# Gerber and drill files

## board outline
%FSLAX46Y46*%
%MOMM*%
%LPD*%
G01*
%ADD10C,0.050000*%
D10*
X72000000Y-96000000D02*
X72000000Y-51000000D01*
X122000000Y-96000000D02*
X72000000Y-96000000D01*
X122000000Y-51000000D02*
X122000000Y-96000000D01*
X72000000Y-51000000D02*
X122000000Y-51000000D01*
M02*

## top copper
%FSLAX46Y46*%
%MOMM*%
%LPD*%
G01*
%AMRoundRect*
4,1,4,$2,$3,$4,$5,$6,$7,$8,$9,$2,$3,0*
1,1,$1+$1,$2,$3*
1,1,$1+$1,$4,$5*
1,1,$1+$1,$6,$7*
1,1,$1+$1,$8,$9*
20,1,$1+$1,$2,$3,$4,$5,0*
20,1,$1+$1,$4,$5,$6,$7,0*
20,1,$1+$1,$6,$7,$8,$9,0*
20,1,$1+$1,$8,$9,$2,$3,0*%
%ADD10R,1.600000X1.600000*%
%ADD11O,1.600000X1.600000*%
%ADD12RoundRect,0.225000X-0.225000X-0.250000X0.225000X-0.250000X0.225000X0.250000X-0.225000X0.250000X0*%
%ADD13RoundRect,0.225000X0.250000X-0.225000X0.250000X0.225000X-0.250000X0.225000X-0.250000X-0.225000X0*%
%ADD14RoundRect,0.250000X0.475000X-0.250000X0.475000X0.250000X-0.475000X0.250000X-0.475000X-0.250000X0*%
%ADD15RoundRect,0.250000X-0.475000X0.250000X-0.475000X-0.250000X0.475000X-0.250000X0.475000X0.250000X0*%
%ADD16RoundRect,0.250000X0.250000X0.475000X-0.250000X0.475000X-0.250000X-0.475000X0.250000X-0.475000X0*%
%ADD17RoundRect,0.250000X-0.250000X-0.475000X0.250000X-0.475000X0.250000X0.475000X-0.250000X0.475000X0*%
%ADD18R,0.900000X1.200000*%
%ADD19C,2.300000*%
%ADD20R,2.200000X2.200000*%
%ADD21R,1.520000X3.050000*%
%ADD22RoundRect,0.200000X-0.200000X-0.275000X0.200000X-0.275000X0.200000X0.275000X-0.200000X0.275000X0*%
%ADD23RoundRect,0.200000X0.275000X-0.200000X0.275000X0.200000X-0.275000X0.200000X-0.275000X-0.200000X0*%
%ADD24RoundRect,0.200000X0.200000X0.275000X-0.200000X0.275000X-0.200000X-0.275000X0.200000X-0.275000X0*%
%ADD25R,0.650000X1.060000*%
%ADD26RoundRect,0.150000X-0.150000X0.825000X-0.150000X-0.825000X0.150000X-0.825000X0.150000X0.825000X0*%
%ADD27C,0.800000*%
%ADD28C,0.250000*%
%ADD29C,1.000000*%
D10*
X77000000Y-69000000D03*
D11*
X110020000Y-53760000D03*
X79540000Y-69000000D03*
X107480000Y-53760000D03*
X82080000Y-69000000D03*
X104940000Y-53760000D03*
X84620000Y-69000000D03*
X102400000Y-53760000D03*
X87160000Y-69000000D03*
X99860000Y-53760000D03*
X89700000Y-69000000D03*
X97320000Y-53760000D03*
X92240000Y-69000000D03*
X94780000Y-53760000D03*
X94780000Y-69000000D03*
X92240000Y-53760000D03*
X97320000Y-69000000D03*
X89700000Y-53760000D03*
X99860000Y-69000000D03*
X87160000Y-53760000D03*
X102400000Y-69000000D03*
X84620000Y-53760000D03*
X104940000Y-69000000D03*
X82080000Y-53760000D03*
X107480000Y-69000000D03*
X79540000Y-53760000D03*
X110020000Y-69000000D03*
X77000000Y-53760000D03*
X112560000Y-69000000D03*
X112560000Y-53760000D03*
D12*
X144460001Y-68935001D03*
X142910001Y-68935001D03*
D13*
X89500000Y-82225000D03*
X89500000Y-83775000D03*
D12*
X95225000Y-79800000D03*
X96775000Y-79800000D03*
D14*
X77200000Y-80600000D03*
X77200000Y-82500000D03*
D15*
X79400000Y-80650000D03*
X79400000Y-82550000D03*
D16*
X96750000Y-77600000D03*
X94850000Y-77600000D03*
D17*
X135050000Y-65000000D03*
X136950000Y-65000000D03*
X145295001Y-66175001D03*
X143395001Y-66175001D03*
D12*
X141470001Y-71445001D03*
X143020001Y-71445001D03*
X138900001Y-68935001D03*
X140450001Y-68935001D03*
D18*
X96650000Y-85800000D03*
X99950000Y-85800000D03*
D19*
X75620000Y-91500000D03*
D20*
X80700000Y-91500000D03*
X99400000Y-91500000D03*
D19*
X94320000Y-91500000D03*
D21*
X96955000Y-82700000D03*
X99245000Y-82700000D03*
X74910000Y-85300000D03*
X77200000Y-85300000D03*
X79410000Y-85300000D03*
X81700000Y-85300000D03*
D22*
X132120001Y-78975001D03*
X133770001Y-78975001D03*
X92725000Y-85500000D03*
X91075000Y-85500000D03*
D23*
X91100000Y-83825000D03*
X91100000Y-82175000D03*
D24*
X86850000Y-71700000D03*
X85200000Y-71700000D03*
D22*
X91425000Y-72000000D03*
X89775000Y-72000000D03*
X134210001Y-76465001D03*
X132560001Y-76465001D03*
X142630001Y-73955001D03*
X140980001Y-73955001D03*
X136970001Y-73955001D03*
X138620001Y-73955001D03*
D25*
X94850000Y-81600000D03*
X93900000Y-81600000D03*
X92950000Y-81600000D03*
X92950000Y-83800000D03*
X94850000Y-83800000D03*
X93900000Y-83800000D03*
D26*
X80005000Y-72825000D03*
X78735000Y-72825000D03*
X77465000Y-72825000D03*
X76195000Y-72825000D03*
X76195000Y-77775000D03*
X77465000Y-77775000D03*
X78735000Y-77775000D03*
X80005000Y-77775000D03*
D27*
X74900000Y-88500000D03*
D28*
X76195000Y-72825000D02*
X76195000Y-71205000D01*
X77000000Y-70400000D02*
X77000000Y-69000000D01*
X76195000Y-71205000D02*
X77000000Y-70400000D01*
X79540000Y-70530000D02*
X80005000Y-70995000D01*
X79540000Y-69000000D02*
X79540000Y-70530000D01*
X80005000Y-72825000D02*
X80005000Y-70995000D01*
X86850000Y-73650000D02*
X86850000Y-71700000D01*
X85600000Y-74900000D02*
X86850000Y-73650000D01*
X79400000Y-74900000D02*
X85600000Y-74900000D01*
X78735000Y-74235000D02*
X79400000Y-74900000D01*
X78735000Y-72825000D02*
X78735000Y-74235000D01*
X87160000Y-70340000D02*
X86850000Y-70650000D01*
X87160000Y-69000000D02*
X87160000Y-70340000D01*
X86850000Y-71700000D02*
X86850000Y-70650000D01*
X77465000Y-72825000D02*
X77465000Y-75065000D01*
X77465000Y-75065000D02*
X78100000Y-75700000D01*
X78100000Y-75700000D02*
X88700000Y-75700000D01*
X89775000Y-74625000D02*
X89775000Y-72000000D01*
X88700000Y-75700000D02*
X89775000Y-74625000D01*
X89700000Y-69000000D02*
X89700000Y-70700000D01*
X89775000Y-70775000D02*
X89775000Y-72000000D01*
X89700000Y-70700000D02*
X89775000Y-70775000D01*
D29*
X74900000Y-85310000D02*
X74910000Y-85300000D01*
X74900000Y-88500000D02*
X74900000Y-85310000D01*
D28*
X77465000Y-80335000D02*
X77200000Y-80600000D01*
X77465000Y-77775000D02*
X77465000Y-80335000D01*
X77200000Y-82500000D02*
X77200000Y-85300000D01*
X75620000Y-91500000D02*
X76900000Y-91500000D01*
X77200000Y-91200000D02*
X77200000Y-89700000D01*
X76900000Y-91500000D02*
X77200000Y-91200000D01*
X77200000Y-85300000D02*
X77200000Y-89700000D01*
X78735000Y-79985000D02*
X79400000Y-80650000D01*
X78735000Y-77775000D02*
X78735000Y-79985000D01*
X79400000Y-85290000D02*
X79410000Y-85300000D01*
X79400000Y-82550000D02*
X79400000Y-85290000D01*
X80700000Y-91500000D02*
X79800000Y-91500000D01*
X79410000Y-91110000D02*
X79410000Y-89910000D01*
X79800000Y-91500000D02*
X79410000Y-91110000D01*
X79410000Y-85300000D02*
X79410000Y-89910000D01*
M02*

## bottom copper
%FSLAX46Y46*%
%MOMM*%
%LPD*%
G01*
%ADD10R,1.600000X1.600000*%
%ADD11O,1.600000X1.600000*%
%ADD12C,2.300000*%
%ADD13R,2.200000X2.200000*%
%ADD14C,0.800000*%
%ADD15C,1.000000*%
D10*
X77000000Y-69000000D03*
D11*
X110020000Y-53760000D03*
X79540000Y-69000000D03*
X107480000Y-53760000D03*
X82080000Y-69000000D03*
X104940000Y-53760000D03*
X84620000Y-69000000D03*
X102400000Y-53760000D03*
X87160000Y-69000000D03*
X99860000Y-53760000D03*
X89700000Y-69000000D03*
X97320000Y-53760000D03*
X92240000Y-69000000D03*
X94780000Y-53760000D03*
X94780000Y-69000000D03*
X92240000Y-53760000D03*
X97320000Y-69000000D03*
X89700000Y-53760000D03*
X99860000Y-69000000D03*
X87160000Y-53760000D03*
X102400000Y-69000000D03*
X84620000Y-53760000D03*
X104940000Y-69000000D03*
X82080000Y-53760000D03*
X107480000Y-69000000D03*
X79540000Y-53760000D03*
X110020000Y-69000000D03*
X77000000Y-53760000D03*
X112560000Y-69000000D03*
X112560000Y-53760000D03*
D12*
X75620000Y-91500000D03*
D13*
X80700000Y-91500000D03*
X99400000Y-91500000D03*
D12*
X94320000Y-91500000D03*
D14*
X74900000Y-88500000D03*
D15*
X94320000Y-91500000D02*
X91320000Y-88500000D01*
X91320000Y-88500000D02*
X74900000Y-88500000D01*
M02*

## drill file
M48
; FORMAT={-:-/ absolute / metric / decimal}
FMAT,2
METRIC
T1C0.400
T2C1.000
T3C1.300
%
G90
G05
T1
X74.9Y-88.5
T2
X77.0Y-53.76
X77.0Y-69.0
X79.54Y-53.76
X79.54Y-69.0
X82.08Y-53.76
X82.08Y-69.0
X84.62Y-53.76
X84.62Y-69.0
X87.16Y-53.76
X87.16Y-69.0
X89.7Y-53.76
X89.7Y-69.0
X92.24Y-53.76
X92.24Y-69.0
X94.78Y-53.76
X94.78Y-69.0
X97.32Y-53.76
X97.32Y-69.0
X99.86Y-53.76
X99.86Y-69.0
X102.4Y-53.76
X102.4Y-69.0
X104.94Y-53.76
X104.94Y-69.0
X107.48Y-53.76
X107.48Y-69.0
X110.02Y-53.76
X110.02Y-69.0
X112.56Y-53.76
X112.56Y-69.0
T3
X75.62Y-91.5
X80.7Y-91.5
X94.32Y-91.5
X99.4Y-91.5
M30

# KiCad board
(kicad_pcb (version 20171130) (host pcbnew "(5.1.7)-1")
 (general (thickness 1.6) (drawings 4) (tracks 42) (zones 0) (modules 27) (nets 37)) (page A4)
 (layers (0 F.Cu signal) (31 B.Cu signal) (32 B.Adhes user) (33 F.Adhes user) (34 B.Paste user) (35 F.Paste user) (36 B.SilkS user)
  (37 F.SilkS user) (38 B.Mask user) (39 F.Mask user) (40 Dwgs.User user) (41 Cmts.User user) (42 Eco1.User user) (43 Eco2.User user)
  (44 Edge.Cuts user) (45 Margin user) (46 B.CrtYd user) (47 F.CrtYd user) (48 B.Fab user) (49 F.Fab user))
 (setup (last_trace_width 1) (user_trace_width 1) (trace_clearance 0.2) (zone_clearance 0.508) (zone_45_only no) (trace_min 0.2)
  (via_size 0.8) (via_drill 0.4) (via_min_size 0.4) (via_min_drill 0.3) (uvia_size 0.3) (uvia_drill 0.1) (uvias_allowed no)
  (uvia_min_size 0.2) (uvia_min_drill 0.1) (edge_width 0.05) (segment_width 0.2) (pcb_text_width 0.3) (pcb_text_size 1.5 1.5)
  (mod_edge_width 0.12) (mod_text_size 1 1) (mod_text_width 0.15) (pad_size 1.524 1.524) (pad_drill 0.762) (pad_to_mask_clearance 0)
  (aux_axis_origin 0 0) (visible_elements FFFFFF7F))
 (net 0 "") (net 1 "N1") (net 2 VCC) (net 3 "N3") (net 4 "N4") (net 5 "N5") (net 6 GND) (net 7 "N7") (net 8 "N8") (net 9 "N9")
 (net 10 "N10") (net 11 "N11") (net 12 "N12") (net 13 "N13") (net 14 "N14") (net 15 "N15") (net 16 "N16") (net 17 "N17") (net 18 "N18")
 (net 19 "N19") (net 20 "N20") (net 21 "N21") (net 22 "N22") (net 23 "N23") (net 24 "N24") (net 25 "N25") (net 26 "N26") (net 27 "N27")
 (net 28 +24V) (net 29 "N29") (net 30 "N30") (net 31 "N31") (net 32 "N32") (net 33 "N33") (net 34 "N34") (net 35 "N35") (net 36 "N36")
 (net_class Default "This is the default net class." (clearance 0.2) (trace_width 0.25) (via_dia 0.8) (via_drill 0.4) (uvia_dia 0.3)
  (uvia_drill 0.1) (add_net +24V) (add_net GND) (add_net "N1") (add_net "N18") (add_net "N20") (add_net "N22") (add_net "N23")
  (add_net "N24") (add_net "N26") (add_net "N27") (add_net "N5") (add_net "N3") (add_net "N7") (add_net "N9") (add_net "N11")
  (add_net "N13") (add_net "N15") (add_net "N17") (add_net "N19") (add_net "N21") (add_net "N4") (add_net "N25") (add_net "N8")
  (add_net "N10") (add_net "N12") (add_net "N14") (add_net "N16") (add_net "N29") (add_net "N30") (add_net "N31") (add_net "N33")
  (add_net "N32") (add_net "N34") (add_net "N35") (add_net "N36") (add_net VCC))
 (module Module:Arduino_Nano (layer F.Cu) (at 77 69 90)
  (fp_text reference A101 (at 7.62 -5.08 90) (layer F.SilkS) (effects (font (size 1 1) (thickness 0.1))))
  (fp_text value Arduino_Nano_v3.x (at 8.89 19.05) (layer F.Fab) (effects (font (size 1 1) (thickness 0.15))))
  (pad 1 thru_hole rect (at 0 0 90) (size 1.6 1.6) (drill 1) (layers *.Cu *.Mask) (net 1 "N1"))
  (pad 17 thru_hole oval (at 15.24 33.02 90) (size 1.6 1.6) (drill 1) (layers *.Cu *.Mask) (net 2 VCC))
  (pad 2 thru_hole oval (at 0 2.54 90) (size 1.6 1.6) (drill 1) (layers *.Cu *.Mask) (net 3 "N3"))
  (pad 18 thru_hole oval (at 15.24 30.48 90) (size 1.6 1.6) (drill 1) (layers *.Cu *.Mask) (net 2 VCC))
  (pad 3 thru_hole oval (at 0 5.08 90) (size 1.6 1.6) (drill 1) (layers *.Cu *.Mask) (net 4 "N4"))
  (pad 19 thru_hole oval (at 15.24 27.94 90) (size 1.6 1.6) (drill 1) (layers *.Cu *.Mask) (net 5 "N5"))
  (pad 4 thru_hole oval (at 0 7.62 90) (size 1.6 1.6) (drill 1) (layers *.Cu *.Mask) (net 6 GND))
  (pad 20 thru_hole oval (at 15.24 25.4 90) (size 1.6 1.6) (drill 1) (layers *.Cu *.Mask) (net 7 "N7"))
  (pad 5 thru_hole oval (at 0 10.16 90) (size 1.6 1.6) (drill 1) (layers *.Cu *.Mask) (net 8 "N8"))
  (pad 21 thru_hole oval (at 15.24 22.86 90) (size 1.6 1.6) (drill 1) (layers *.Cu *.Mask) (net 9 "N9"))
  (pad 6 thru_hole oval (at 0 12.7 90) (size 1.6 1.6) (drill 1) (layers *.Cu *.Mask) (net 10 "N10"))
  (pad 22 thru_hole oval (at 15.24 20.32 90) (size 1.6 1.6) (drill 1) (layers *.Cu *.Mask) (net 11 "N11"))
  (pad 7 thru_hole oval (at 0 15.24 90) (size 1.6 1.6) (drill 1) (layers *.Cu *.Mask) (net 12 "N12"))
  (pad 23 thru_hole oval (at 15.24 17.78 90) (size 1.6 1.6) (drill 1) (layers *.Cu *.Mask) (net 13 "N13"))
  (pad 8 thru_hole oval (at 0 17.78 90) (size 1.6 1.6) (drill 1) (layers *.Cu *.Mask) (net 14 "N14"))
  (pad 24 thru_hole oval (at 15.24 15.24 90) (size 1.6 1.6) (drill 1) (layers *.Cu *.Mask) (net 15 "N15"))
  (pad 9 thru_hole oval (at 0 20.32 90) (size 1.6 1.6) (drill 1) (layers *.Cu *.Mask) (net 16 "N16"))
  (pad 25 thru_hole oval (at 15.24 12.7 90) (size 1.6 1.6) (drill 1) (layers *.Cu *.Mask) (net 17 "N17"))
  (pad 10 thru_hole oval (at 0 22.86 90) (size 1.6 1.6) (drill 1) (layers *.Cu *.Mask) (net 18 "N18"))
  (pad 26 thru_hole oval (at 15.24 10.16 90) (size 1.6 1.6) (drill 1) (layers *.Cu *.Mask) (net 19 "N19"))
  (pad 11 thru_hole oval (at 0 25.4 90) (size 1.6 1.6) (drill 1) (layers *.Cu *.Mask) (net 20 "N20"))
  (pad 27 thru_hole oval (at 15.24 7.62 90) (size 1.6 1.6) (drill 1) (layers *.Cu *.Mask) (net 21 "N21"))
  (pad 12 thru_hole oval (at 0 27.94 90) (size 1.6 1.6) (drill 1) (layers *.Cu *.Mask) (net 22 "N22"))
  (pad 28 thru_hole oval (at 15.24 5.08 90) (size 1.6 1.6) (drill 1) (layers *.Cu *.Mask) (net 4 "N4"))
  (pad 13 thru_hole oval (at 0 30.48 90) (size 1.6 1.6) (drill 1) (layers *.Cu *.Mask) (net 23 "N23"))
  (pad 29 thru_hole oval (at 15.24 2.54 90) (size 1.6 1.6) (drill 1) (layers *.Cu *.Mask) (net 6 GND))
  (pad 14 thru_hole oval (at 0 33.02 90) (size 1.6 1.6) (drill 1) (layers *.Cu *.Mask) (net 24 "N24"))
  (pad 30 thru_hole oval (at 15.24 0 90) (size 1.6 1.6) (drill 1) (layers *.Cu *.Mask) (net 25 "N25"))
  (pad 15 thru_hole oval (at 0 35.56 90) (size 1.6 1.6) (drill 1) (layers *.Cu *.Mask) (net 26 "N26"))
  (pad 16 thru_hole oval (at 15.24 35.56 90) (size 1.6 1.6) (drill 1) (layers *.Cu *.Mask) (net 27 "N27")))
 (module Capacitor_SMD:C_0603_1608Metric (layer F.Cu) (at 143.685001 68.935001)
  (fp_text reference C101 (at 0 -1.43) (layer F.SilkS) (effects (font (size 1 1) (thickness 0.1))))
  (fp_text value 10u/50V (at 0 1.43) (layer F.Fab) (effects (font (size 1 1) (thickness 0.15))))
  (pad 2 smd roundrect (at 0.775 0) (size 0.9 0.95) (layers F.Cu F.Paste F.Mask) (roundrect_rratio 0.25) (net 6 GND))
  (pad 1 smd roundrect (at -0.775 0) (size 0.9 0.95) (layers F.Cu F.Paste F.Mask) (roundrect_rratio 0.25) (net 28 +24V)))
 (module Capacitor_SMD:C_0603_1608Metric (layer F.Cu) (at 89.5 83 90)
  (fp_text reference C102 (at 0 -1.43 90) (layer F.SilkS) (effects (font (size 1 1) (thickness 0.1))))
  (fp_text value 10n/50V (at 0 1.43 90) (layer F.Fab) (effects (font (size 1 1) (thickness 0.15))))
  (pad 2 smd roundrect (at 0.775 0 90) (size 0.9 0.95) (layers F.Cu F.Paste F.Mask) (roundrect_rratio 0.25) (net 6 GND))
  (pad 1 smd roundrect (at -0.775 0 90) (size 0.9 0.95) (layers F.Cu F.Paste F.Mask) (roundrect_rratio 0.25) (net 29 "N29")))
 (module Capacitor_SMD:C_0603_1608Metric (layer F.Cu) (at 96 79.8)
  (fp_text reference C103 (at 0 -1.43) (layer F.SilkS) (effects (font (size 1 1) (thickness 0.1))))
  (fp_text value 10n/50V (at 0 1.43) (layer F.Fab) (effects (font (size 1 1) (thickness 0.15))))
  (pad 1 smd roundrect (at -0.775 0) (size 0.9 0.95) (layers F.Cu F.Paste F.Mask) (roundrect_rratio 0.25) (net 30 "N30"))
  (pad 2 smd roundrect (at 0.775 0) (size 0.9 0.95) (layers F.Cu F.Paste F.Mask) (roundrect_rratio 0.25) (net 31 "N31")))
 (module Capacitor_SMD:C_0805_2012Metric (layer F.Cu) (at 77.2 81.55 90)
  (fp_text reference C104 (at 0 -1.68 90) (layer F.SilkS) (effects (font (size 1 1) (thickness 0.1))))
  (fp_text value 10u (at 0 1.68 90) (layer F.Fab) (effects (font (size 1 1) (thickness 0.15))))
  (pad 2 smd roundrect (at 0.95 0 90) (size 1 1.45) (layers F.Cu F.Paste F.Mask) (roundrect_rratio 0.25) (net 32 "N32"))
  (pad 1 smd roundrect (at -0.95 0 90) (size 1 1.45) (layers F.Cu F.Paste F.Mask) (roundrect_rratio 0.25) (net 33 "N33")))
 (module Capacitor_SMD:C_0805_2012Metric (layer F.Cu) (at 79.4 81.6 270)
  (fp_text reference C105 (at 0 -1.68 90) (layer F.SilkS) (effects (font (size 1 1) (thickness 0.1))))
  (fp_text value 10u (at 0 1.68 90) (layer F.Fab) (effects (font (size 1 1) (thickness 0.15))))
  (pad 1 smd roundrect (at -0.95 0 270) (size 1 1.45) (layers F.Cu F.Paste F.Mask) (roundrect_rratio 0.25) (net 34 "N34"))
  (pad 2 smd roundrect (at 0.95 0 270) (size 1 1.45) (layers F.Cu F.Paste F.Mask) (roundrect_rratio 0.25) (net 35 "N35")))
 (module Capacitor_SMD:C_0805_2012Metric (layer F.Cu) (at 95.8 77.6 180)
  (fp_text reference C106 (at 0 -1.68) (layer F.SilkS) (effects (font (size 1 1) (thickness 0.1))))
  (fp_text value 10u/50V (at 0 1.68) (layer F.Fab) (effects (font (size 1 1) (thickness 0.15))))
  (pad 1 smd roundrect (at -0.95 0 180) (size 1 1.45) (layers F.Cu F.Paste F.Mask) (roundrect_rratio 0.25) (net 2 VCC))
  (pad 2 smd roundrect (at 0.95 0 180) (size 1 1.45) (layers F.Cu F.Paste F.Mask) (roundrect_rratio 0.25) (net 6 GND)))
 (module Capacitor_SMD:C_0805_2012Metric (layer F.Cu) (at 136 65)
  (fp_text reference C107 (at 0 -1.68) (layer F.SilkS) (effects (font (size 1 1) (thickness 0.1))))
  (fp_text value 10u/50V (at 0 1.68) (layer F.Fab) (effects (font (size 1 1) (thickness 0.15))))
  (pad 1 smd roundrect (at -0.95 0) (size 1 1.45) (layers F.Cu F.Paste F.Mask) (roundrect_rratio 0.25) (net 28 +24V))
  (pad 2 smd roundrect (at 0.95 0) (size 1 1.45) (layers F.Cu F.Paste F.Mask) (roundrect_rratio 0.25) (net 6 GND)))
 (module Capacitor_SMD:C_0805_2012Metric (layer F.Cu) (at 144.345001 66.175001)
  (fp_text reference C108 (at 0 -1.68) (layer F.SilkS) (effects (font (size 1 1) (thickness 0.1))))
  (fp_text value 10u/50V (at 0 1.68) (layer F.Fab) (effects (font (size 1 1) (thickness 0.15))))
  (pad 2 smd roundrect (at 0.95 0) (size 1 1.45) (layers F.Cu F.Paste F.Mask) (roundrect_rratio 0.25) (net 6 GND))
  (pad 1 smd roundrect (at -0.95 0) (size 1 1.45) (layers F.Cu F.Paste F.Mask) (roundrect_rratio 0.25) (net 2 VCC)))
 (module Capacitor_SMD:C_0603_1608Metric (layer F.Cu) (at 142.245001 71.445001)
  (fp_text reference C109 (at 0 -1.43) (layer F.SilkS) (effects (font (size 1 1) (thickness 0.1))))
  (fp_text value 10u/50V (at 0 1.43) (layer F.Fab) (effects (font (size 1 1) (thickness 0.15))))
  (pad 1 smd roundrect (at -0.775 0) (size 0.9 0.95) (layers F.Cu F.Paste F.Mask) (roundrect_rratio 0.25) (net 28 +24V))
  (pad 2 smd roundrect (at 0.775 0) (size 0.9 0.95) (layers F.Cu F.Paste F.Mask) (roundrect_rratio 0.25) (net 6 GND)))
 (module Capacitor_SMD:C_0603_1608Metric (layer F.Cu) (at 139.675001 68.935001)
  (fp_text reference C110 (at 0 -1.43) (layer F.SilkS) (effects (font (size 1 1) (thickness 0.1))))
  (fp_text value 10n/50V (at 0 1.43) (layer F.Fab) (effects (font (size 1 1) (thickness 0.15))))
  (pad 1 smd roundrect (at -0.775 0) (size 0.9 0.95) (layers F.Cu F.Paste F.Mask) (roundrect_rratio 0.25) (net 2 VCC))
  (pad 2 smd roundrect (at 0.775 0) (size 0.9 0.95) (layers F.Cu F.Paste F.Mask) (roundrect_rratio 0.25) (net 6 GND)))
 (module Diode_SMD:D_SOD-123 (layer F.Cu) (at 98.3 85.8)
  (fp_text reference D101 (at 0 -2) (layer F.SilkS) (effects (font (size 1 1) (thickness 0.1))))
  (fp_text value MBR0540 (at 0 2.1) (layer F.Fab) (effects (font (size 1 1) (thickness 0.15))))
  (pad 1 smd rect (at -1.65 0) (size 0.9 1.2) (layers F.Cu F.Paste F.Mask) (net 31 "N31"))
  (pad 2 smd rect (at 1.65 0) (size 0.9 1.2) (layers F.Cu F.Paste F.Mask) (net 6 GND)))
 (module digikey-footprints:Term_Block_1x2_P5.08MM (layer F.Cu) (at 80.7 91.5 180)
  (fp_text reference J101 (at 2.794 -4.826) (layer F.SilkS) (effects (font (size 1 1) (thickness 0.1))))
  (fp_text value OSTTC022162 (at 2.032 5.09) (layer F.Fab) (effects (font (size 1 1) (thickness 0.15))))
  (pad 2 thru_hole circle (at 5.08 0 180) (size 2.3 2.3) (drill 1.3) (layers *.Cu *.Mask) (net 33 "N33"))
  (pad 1 thru_hole rect (at 0 0 180) (size 2.2 2.2) (drill 1.3) (layers *.Cu *.Mask) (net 35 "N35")))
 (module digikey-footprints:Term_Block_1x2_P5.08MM (layer F.Cu) (at 99.4 91.5 180)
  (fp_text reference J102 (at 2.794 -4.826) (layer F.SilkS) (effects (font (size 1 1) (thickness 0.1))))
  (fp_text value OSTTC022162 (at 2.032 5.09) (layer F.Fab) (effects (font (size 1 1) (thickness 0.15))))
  (pad 1 thru_hole rect (at 0 0 180) (size 2.2 2.2) (drill 1.3) (layers *.Cu *.Mask) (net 6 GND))
  (pad 2 thru_hole circle (at 5.08 0 180) (size 2.3 2.3) (drill 1.3) (layers *.Cu *.Mask) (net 28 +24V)))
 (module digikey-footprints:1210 (layer F.Cu) (at 98.1 82.7 180)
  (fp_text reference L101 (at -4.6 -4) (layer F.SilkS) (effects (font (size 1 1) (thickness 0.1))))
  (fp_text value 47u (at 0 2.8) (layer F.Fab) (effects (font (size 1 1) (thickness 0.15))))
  (pad 2 smd rect (at 1.145 0 180) (size 1.52 3.05) (layers F.Cu F.Paste F.Mask) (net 31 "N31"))
  (pad 1 smd rect (at -1.145 0 180) (size 1.52 3.05) (layers F.Cu F.Paste F.Mask) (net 2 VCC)))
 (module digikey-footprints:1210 (layer F.Cu) (at 76.055 85.3)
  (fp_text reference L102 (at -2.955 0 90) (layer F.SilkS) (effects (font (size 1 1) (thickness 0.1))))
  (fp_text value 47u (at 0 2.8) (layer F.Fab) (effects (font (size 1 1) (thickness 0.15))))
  (pad 1 smd rect (at -1.145 0) (size 1.52 3.05) (layers F.Cu F.Paste F.Mask) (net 28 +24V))
  (pad 2 smd rect (at 1.145 0) (size 1.52 3.05) (layers F.Cu F.Paste F.Mask) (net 33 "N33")))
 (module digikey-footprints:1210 (layer F.Cu) (at 80.555 85.3)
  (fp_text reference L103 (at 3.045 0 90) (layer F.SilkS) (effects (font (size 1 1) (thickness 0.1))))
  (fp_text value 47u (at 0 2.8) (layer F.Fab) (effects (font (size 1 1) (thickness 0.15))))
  (pad 1 smd rect (at -1.145 0) (size 1.52 3.05) (layers F.Cu F.Paste F.Mask) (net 35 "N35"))
  (pad 2 smd rect (at 1.145 0) (size 1.52 3.05) (layers F.Cu F.Paste F.Mask) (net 6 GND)))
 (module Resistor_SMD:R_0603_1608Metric (layer F.Cu) (at 132.945001 78.975001)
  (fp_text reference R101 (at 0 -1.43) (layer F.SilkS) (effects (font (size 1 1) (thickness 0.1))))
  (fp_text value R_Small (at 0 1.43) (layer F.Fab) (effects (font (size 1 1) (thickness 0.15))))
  (pad 1 smd roundrect (at -0.825 0) (size 0.8 0.95) (layers F.Cu F.Paste F.Mask) (roundrect_rratio 0.25) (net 4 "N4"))
  (pad 2 smd roundrect (at 0.825 0) (size 0.8 0.95) (layers F.Cu F.Paste F.Mask) (roundrect_rratio 0.25) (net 2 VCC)))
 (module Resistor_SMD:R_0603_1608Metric (layer F.Cu) (at 91.9 85.5)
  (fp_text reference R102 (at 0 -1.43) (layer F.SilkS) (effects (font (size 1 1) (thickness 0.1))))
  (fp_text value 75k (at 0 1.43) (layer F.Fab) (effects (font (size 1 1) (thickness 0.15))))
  (pad 2 smd roundrect (at 0.825 0) (size 0.8 0.95) (layers F.Cu F.Paste F.Mask) (roundrect_rratio 0.25) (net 28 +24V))
  (pad 1 smd roundrect (at -0.825 0) (size 0.8 0.95) (layers F.Cu F.Paste F.Mask) (roundrect_rratio 0.25) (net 29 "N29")))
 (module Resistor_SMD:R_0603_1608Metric (layer F.Cu) (at 91.1 83 90)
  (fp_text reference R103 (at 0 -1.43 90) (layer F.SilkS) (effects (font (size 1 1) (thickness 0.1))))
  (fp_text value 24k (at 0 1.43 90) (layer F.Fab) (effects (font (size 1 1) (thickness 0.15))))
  (pad 1 smd roundrect (at -0.825 0 90) (size 0.8 0.95) (layers F.Cu F.Paste F.Mask) (roundrect_rratio 0.25) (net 29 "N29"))
  (pad 2 smd roundrect (at 0.825 0 90) (size 0.8 0.95) (layers F.Cu F.Paste F.Mask) (roundrect_rratio 0.25) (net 6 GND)))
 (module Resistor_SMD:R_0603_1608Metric (layer F.Cu) (at 86.025 71.7 180)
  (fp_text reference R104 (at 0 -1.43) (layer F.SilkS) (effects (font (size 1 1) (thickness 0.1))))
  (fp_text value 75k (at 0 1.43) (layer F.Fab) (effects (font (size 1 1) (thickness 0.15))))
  (pad 1 smd roundrect (at -0.825 0 180) (size 0.8 0.95) (layers F.Cu F.Paste F.Mask) (roundrect_rratio 0.25) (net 8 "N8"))
  (pad 2 smd roundrect (at 0.825 0 180) (size 0.8 0.95) (layers F.Cu F.Paste F.Mask) (roundrect_rratio 0.25) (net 6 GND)))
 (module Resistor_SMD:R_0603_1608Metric (layer F.Cu) (at 90.6 72)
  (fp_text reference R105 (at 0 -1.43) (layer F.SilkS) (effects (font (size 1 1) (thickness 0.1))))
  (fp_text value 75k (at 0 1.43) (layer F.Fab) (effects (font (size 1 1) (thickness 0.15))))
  (pad 2 smd roundrect (at 0.825 0) (size 0.8 0.95) (layers F.Cu F.Paste F.Mask) (roundrect_rratio 0.25) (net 6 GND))
  (pad 1 smd roundrect (at -0.825 0) (size 0.8 0.95) (layers F.Cu F.Paste F.Mask) (roundrect_rratio 0.25) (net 10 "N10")))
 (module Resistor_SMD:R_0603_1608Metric (layer F.Cu) (at 133.385001 76.465001)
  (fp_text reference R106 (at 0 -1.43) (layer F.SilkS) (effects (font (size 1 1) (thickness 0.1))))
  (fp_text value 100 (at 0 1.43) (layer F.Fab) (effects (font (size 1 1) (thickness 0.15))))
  (pad 2 smd roundrect (at 0.825 0) (size 0.8 0.95) (layers F.Cu F.Paste F.Mask) (roundrect_rratio 0.25) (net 32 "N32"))
  (pad 1 smd roundrect (at -0.825 0) (size 0.8 0.95) (layers F.Cu F.Paste F.Mask) (roundrect_rratio 0.25) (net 34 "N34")))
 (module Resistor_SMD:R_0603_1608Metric (layer F.Cu) (at 141.805001 73.955001)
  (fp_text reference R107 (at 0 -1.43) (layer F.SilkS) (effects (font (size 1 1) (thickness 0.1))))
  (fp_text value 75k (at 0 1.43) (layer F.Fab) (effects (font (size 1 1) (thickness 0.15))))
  (pad 2 smd roundrect (at 0.825 0) (size 0.8 0.95) (layers F.Cu F.Paste F.Mask) (roundrect_rratio 0.25) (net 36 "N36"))
  (pad 1 smd roundrect (at -0.825 0) (size 0.8 0.95) (layers F.Cu F.Paste F.Mask) (roundrect_rratio 0.25) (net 2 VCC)))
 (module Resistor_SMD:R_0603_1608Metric (layer F.Cu) (at 137.795001 73.955001)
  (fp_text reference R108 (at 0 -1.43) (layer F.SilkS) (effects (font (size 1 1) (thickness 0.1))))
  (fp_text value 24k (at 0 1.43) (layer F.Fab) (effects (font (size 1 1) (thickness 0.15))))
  (pad 1 smd roundrect (at -0.825 0) (size 0.8 0.95) (layers F.Cu F.Paste F.Mask) (roundrect_rratio 0.25) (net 36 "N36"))
  (pad 2 smd roundrect (at 0.825 0) (size 0.8 0.95) (layers F.Cu F.Paste F.Mask) (roundrect_rratio 0.25) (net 6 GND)))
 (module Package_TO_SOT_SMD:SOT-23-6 (layer F.Cu) (at 93.9 82.7 270)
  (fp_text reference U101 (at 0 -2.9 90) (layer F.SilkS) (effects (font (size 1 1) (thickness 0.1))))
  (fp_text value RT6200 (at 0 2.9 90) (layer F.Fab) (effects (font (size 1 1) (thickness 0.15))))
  (pad 1 smd rect (at -1.1 -0.95 270) (size 1.06 0.65) (layers F.Cu F.Paste F.Mask) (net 30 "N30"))
  (pad 2 smd rect (at -1.1 0 270) (size 1.06 0.65) (layers F.Cu F.Paste F.Mask) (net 6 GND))
  (pad 3 smd rect (at -1.1 0.95 270) (size 1.06 0.65) (layers F.Cu F.Paste F.Mask) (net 36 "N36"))
  (pad 4 smd rect (at 1.1 0.95 270) (size 1.06 0.65) (layers F.Cu F.Paste F.Mask) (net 29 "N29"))
  (pad 6 smd rect (at 1.1 -0.95 270) (size 1.06 0.65) (layers F.Cu F.Paste F.Mask) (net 31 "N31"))
  (pad 5 smd rect (at 1.1 0 270) (size 1.06 0.65) (layers F.Cu F.Paste F.Mask) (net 28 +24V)))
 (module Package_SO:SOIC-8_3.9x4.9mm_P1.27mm (layer F.Cu) (at 78.1 75.3 270)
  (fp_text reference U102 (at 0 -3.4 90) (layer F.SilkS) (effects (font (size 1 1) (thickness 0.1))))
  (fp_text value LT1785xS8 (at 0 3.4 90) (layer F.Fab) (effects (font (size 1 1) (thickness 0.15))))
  (pad 1 smd roundrect (at -2.475 -1.905 270) (size 1.95 0.6) (layers F.Cu F.Paste F.Mask) (roundrect_rratio 0.25) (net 3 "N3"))
  (pad 2 smd roundrect (at -2.475 -0.635 270) (size 1.95 0.6) (layers F.Cu F.Paste F.Mask) (roundrect_rratio 0.25) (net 8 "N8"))
  (pad 3 smd roundrect (at -2.475 0.635 270) (size 1.95 0.6) (layers F.Cu F.Paste F.Mask) (roundrect_rratio 0.25) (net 10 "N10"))
  (pad 4 smd roundrect (at -2.475 1.905 270) (size 1.95 0.6) (layers F.Cu F.Paste F.Mask) (roundrect_rratio 0.25) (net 1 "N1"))
  (pad 5 smd roundrect (at 2.475 1.905 270) (size 1.95 0.6) (layers F.Cu F.Paste F.Mask) (roundrect_rratio 0.25) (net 6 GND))
  (pad 6 smd roundrect (at 2.475 0.635 270) (size 1.95 0.6) (layers F.Cu F.Paste F.Mask) (roundrect_rratio 0.25) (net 32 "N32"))
  (pad 7 smd roundrect (at 2.475 -0.635 270) (size 1.95 0.6) (layers F.Cu F.Paste F.Mask) (roundrect_rratio 0.25) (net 34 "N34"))
  (pad 8 smd roundrect (at 2.475 -1.905 270) (size 1.95 0.6) (layers F.Cu F.Paste F.Mask) (roundrect_rratio 0.25) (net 2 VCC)))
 (gr_line (start 72 96) (end 72 51) (layer Edge.Cuts) (width 0.05))
 (gr_line (start 122 96) (end 72 96) (layer Edge.Cuts) (width 0.05))
 (gr_line (start 122 51) (end 122 96) (layer Edge.Cuts) (width 0.05))
 (gr_line (start 72 51) (end 122 51) (layer Edge.Cuts) (width 0.05))
 (segment (start 76.195 72.825) (end 76.195 71.205) (width 0.25) (layer F.Cu) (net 1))
 (segment (start 77 70.4) (end 77 69) (width 0.25) (layer F.Cu) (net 1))
 (segment (start 76.195 71.205) (end 77 70.4) (width 0.25) (layer F.Cu) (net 1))
 (segment (start 79.54 70.53) (end 80.005 70.995) (width 0.25) (layer F.Cu) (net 3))
 (segment (start 79.54 69) (end 79.54 70.53) (width 0.25) (layer F.Cu) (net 3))
 (segment (start 80.005 72.825) (end 80.005 70.995) (width 0.25) (layer F.Cu) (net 3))
 (segment (start 86.85 73.65) (end 86.85 71.7) (width 0.25) (layer F.Cu) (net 8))
 (segment (start 85.6 74.9) (end 86.85 73.65) (width 0.25) (layer F.Cu) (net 8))
 (segment (start 79.4 74.9) (end 85.6 74.9) (width 0.25) (layer F.Cu) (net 8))
 (segment (start 78.735 74.235) (end 79.4 74.9) (width 0.25) (layer F.Cu) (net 8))
 (segment (start 78.735 72.825) (end 78.735 74.235) (width 0.25) (layer F.Cu) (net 8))
 (segment (start 87.16 70.34) (end 86.85 70.65) (width 0.25) (layer F.Cu) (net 8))
 (segment (start 87.16 69) (end 87.16 70.34) (width 0.25) (layer F.Cu) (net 8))
 (segment (start 86.85 71.7) (end 86.85 70.65) (width 0.25) (layer F.Cu) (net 8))
 (segment (start 77.465 72.825) (end 77.465 75.065) (width 0.25) (layer F.Cu) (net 10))
 (segment (start 77.465 75.065) (end 78.1 75.7) (width 0.25) (layer F.Cu) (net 10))
 (segment (start 78.1 75.7) (end 88.7 75.7) (width 0.25) (layer F.Cu) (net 10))
 (segment (start 89.775 74.625) (end 89.775 72) (width 0.25) (layer F.Cu) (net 10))
 (segment (start 88.7 75.7) (end 89.775 74.625) (width 0.25) (layer F.Cu) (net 10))
 (segment (start 89.7 69) (end 89.7 70.7) (width 0.25) (layer F.Cu) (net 10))
 (segment (start 89.775 70.775) (end 89.775 72) (width 0.25) (layer F.Cu) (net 10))
 (segment (start 89.7 70.7) (end 89.775 70.775) (width 0.25) (layer F.Cu) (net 10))
 (segment (start 94.32 91.5) (end 91.32 88.5) (width 1) (layer B.Cu) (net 28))
 (via (at 74.9 88.5) (size 0.8) (drill 0.4) (layers F.Cu B.Cu) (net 28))
 (segment (start 91.32 88.5) (end 74.9 88.5) (width 1) (layer B.Cu) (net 28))
 (segment (start 74.9 85.31) (end 74.91 85.3) (width 1) (layer F.Cu) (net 28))
 (segment (start 74.9 88.5) (end 74.9 85.31) (width 1) (layer F.Cu) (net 28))
 (segment (start 77.465 80.335) (end 77.2 80.6) (width 0.25) (layer F.Cu) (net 32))
 (segment (start 77.465 77.775) (end 77.465 80.335) (width 0.25) (layer F.Cu) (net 32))
 (segment (start 77.2 82.5) (end 77.2 85.3) (width 0.25) (layer F.Cu) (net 33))
 (segment (start 75.62 91.5) (end 76.9 91.5) (width 0.25) (layer F.Cu) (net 33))
 (segment (start 77.2 91.2) (end 77.2 89.7) (width 0.25) (layer F.Cu) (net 33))
 (segment (start 76.9 91.5) (end 77.2 91.2) (width 0.25) (layer F.Cu) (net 33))
 (segment (start 77.2 85.3) (end 77.2 89.7) (width 0.25) (layer F.Cu) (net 33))
 (segment (start 78.735 79.985) (end 79.4 80.65) (width 0.25) (layer F.Cu) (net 34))
 (segment (start 78.735 77.775) (end 78.735 79.985) (width 0.25) (layer F.Cu) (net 34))
 (segment (start 79.4 85.29) (end 79.41 85.3) (width 0.25) (layer F.Cu) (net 35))
 (segment (start 79.4 82.55) (end 79.4 85.29) (width 0.25) (layer F.Cu) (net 35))
 (segment (start 80.7 91.5) (end 79.8 91.5) (width 0.25) (layer F.Cu) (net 35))
 (segment (start 79.41 91.11) (end 79.41 89.91) (width 0.25) (layer F.Cu) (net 35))
 (segment (start 79.8 91.5) (end 79.41 91.11) (width 0.25) (layer F.Cu) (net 35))
 (segment (start 79.41 85.3) (end 79.41 89.91) (width 0.25) (layer F.Cu) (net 35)))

